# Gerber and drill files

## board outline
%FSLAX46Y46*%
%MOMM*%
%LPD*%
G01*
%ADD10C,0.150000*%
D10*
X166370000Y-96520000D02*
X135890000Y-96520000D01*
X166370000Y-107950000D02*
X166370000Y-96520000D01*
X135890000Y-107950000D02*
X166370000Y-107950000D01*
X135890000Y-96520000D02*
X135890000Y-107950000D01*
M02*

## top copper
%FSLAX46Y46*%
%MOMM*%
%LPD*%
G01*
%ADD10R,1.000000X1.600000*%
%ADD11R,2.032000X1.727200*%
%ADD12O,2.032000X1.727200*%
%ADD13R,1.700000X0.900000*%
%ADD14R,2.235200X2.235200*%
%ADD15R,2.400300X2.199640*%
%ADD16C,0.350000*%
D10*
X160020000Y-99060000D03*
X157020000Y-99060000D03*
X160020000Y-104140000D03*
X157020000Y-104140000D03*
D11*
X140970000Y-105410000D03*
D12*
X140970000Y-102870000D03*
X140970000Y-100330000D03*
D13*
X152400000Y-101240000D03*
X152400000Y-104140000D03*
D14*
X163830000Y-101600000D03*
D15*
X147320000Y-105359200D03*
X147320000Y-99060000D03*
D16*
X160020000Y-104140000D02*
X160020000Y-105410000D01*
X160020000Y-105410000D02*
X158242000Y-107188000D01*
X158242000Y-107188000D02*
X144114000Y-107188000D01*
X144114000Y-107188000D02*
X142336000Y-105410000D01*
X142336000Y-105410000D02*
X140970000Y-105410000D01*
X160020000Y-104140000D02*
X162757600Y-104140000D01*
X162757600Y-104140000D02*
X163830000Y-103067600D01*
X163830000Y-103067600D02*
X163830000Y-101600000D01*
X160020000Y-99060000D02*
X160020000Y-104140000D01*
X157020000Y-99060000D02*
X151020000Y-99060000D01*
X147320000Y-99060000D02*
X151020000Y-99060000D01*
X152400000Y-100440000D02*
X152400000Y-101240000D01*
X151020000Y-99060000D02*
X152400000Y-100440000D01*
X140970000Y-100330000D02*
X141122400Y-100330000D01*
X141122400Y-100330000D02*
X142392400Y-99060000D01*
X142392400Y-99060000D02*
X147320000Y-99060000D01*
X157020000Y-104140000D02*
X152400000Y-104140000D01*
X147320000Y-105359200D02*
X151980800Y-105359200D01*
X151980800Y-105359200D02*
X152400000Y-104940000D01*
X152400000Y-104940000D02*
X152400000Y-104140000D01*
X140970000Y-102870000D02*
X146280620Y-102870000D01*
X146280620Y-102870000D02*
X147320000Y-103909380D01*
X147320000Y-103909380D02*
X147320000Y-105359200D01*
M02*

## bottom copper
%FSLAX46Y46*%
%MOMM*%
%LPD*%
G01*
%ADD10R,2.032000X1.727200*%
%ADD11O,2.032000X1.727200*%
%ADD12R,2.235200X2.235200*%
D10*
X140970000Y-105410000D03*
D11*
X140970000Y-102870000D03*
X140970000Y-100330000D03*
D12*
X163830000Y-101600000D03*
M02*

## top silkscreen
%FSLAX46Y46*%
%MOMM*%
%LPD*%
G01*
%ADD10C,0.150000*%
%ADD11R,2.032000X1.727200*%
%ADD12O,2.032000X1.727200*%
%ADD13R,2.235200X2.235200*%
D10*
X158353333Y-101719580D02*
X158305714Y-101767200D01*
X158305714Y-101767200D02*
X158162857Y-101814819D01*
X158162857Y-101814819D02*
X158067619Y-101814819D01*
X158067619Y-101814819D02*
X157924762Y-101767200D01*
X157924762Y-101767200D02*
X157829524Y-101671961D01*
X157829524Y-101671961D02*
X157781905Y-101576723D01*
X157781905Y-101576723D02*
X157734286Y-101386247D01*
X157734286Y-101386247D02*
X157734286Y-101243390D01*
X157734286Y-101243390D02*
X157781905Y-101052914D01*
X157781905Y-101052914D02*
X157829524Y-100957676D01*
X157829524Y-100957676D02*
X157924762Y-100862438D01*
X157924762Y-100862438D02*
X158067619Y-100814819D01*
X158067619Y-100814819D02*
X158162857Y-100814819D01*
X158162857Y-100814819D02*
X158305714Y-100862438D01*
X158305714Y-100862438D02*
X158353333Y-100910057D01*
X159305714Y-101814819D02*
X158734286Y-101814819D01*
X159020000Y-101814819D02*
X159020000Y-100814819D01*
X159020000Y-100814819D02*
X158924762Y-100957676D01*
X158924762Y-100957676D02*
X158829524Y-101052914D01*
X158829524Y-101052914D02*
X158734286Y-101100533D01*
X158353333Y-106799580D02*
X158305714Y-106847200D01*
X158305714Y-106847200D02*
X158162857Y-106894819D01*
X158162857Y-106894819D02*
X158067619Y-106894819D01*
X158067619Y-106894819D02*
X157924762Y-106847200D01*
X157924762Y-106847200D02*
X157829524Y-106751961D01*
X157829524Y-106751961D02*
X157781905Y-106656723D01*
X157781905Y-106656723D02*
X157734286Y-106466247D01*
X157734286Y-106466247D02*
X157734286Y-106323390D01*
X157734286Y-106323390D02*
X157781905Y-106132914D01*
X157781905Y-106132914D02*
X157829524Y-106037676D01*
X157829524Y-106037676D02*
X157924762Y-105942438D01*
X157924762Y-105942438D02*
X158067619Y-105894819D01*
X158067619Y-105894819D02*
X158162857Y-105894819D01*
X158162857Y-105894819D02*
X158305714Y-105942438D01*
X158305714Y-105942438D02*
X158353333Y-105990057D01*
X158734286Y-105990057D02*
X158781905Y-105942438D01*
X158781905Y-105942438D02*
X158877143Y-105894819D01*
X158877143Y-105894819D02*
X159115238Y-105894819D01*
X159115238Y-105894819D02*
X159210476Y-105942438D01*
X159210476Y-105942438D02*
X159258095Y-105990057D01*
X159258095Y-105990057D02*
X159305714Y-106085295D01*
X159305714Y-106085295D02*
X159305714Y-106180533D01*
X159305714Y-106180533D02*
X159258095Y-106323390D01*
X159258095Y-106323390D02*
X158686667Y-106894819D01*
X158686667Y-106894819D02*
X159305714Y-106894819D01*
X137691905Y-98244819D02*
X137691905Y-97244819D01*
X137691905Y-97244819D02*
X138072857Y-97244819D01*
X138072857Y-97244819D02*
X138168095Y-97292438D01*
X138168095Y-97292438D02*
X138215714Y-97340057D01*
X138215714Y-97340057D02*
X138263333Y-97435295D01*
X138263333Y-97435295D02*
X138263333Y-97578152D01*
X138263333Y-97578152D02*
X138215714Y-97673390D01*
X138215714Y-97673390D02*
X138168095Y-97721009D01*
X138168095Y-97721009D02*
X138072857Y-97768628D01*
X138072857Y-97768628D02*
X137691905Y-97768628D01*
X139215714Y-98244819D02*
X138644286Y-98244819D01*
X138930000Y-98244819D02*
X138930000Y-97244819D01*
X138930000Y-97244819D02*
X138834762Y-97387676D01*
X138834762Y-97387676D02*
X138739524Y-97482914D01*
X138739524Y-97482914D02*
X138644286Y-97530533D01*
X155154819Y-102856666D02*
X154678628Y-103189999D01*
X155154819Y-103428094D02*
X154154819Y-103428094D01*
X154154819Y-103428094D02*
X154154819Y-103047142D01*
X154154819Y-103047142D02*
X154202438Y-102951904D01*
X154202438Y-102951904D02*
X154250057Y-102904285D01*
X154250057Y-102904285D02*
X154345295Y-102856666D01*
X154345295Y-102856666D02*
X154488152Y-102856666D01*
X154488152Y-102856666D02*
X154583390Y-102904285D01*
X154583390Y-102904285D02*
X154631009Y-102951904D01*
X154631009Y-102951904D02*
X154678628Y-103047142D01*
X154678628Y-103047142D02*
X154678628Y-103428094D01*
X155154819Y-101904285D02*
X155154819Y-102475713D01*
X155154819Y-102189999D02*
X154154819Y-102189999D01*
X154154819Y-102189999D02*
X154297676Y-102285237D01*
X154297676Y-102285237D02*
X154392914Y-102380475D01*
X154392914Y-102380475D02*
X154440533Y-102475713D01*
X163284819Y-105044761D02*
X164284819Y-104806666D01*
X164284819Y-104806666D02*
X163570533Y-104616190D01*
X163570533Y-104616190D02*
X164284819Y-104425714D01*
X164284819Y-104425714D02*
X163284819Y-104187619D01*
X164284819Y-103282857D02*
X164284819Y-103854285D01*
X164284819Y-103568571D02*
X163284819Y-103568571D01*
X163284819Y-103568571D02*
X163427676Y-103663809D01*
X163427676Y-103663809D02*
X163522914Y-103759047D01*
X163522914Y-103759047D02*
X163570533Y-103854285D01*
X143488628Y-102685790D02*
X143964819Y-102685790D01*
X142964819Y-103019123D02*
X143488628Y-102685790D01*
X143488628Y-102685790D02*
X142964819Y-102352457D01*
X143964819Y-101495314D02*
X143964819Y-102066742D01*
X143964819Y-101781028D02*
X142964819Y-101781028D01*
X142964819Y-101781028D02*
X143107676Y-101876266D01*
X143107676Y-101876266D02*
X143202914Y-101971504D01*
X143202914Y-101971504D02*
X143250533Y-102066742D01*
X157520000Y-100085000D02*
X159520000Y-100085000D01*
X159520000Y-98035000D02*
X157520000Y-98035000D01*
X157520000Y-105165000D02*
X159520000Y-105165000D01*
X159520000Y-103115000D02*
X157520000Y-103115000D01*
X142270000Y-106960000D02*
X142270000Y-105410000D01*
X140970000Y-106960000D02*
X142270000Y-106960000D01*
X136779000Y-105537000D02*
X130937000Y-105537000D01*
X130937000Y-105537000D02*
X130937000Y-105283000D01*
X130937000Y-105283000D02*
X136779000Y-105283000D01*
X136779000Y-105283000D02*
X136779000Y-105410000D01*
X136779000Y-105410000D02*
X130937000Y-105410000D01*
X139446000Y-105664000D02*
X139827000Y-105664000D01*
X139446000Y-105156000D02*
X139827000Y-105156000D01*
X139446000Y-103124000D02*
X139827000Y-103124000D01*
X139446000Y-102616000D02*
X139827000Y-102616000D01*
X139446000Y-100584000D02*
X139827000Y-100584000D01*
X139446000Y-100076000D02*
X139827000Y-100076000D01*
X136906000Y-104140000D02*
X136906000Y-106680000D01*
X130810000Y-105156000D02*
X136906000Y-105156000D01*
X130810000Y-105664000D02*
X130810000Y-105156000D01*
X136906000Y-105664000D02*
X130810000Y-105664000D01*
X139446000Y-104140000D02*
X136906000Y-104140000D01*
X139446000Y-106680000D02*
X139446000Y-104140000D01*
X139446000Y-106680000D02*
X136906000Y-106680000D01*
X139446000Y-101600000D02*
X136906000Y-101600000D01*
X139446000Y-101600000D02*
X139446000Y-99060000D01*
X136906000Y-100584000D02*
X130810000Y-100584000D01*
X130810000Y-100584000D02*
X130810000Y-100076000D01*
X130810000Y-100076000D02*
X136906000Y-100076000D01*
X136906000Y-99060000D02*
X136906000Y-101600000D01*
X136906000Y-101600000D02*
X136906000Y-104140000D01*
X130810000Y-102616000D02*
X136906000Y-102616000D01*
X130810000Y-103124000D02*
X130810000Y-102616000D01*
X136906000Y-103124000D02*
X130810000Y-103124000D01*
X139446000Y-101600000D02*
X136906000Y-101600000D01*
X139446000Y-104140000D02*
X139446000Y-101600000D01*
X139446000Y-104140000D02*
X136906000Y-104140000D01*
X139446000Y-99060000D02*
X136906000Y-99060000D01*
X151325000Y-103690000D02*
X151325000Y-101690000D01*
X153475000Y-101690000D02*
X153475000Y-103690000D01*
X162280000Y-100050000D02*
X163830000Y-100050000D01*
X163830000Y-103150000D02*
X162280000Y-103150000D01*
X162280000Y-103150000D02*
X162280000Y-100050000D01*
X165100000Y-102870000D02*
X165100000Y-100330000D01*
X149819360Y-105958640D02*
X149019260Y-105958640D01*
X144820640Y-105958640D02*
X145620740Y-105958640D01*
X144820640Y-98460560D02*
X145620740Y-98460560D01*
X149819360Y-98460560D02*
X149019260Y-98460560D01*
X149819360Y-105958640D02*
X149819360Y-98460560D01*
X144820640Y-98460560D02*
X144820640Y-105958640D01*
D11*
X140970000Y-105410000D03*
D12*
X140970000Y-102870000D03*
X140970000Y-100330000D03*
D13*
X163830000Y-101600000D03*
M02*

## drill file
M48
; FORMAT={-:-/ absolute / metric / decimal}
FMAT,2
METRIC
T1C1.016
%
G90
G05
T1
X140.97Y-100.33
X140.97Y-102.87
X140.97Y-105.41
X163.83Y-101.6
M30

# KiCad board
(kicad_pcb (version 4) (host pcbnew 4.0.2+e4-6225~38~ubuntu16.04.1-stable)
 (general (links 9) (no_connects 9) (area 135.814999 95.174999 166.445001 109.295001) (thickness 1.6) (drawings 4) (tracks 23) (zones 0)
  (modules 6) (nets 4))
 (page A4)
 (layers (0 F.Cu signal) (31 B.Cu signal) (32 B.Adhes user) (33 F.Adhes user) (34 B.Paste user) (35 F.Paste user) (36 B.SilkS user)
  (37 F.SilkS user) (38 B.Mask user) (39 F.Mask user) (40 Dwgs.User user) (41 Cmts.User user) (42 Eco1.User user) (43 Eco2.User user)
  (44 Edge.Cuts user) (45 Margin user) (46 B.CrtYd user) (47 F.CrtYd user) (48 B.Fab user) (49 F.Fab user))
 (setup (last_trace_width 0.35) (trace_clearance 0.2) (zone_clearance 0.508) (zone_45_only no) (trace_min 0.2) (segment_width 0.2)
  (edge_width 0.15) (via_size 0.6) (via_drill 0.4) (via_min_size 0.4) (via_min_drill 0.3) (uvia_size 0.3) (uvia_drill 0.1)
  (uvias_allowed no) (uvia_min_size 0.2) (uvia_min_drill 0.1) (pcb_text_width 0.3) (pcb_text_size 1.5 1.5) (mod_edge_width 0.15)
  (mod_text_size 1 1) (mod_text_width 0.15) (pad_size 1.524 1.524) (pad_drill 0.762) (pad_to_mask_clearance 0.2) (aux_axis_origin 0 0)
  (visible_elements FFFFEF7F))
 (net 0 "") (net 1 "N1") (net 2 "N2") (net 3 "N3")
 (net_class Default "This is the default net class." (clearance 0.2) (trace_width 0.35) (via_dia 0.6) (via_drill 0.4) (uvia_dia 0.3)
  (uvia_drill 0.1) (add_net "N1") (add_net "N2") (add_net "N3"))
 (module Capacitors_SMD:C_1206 (layer F.Cu) (at 158.52 99.06 180)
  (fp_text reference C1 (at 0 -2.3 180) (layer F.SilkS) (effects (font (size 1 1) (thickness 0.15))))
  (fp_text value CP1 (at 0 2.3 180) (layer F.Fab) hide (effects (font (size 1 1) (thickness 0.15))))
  (fp_line (start 1 -1.025) (end -1 -1.025) (layer F.SilkS) (width 0.15))
  (fp_line (start -1 1.025) (end 1 1.025) (layer F.SilkS) (width 0.15))
  (pad 1 smd rect (at -1.5 0 180) (size 1 1.6) (layers F.Cu F.Paste F.Mask) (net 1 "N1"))
  (pad 2 smd rect (at 1.5 0 180) (size 1 1.6) (layers F.Cu F.Paste F.Mask) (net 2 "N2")))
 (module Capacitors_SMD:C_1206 (layer F.Cu) (at 158.52 104.14 180)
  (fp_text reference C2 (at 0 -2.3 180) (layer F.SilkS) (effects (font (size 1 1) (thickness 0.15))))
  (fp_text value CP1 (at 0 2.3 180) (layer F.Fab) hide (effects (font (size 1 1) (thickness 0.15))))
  (fp_line (start 1 -1.025) (end -1 -1.025) (layer F.SilkS) (width 0.15))
  (fp_line (start -1 1.025) (end 1 1.025) (layer F.SilkS) (width 0.15))
  (pad 1 smd rect (at -1.5 0 180) (size 1 1.6) (layers F.Cu F.Paste F.Mask) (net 1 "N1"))
  (pad 2 smd rect (at 1.5 0 180) (size 1 1.6) (layers F.Cu F.Paste F.Mask) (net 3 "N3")))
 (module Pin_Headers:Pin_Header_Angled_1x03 (layer F.Cu) (at 140.97 105.41 180)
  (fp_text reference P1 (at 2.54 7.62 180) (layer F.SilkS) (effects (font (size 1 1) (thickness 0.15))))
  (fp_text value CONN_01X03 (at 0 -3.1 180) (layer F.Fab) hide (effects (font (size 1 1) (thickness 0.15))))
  (fp_line (start -1.3 -1.55) (end -1.3 0) (layer F.SilkS) (width 0.15))
  (fp_line (start 0 -1.55) (end -1.3 -1.55) (layer F.SilkS) (width 0.15))
  (fp_line (start 4.191 -0.127) (end 10.033 -0.127) (layer F.SilkS) (width 0.15))
  (fp_line (start 10.033 -0.127) (end 10.033 0.127) (layer F.SilkS) (width 0.15))
  (fp_line (start 10.033 0.127) (end 4.191 0.127) (layer F.SilkS) (width 0.15))
  (fp_line (start 4.191 0.127) (end 4.191 0) (layer F.SilkS) (width 0.15))
  (fp_line (start 4.191 0) (end 10.033 0) (layer F.SilkS) (width 0.15))
  (fp_line (start 1.524 -0.254) (end 1.143 -0.254) (layer F.SilkS) (width 0.15))
  (fp_line (start 1.524 0.254) (end 1.143 0.254) (layer F.SilkS) (width 0.15))
  (fp_line (start 1.524 2.286) (end 1.143 2.286) (layer F.SilkS) (width 0.15))
  (fp_line (start 1.524 2.794) (end 1.143 2.794) (layer F.SilkS) (width 0.15))
  (fp_line (start 1.524 4.826) (end 1.143 4.826) (layer F.SilkS) (width 0.15))
  (fp_line (start 1.524 5.334) (end 1.143 5.334) (layer F.SilkS) (width 0.15))
  (fp_line (start 4.064 1.27) (end 4.064 -1.27) (layer F.SilkS) (width 0.15))
  (fp_line (start 10.16 0.254) (end 4.064 0.254) (layer F.SilkS) (width 0.15))
  (fp_line (start 10.16 -0.254) (end 10.16 0.254) (layer F.SilkS) (width 0.15))
  (fp_line (start 4.064 -0.254) (end 10.16 -0.254) (layer F.SilkS) (width 0.15))
  (fp_line (start 1.524 1.27) (end 4.064 1.27) (layer F.SilkS) (width 0.15))
  (fp_line (start 1.524 -1.27) (end 1.524 1.27) (layer F.SilkS) (width 0.15))
  (fp_line (start 1.524 -1.27) (end 4.064 -1.27) (layer F.SilkS) (width 0.15))
  (fp_line (start 1.524 3.81) (end 4.064 3.81) (layer F.SilkS) (width 0.15))
  (fp_line (start 1.524 3.81) (end 1.524 6.35) (layer F.SilkS) (width 0.15))
  (fp_line (start 4.064 4.826) (end 10.16 4.826) (layer F.SilkS) (width 0.15))
  (fp_line (start 10.16 4.826) (end 10.16 5.334) (layer F.SilkS) (width 0.15))
  (fp_line (start 10.16 5.334) (end 4.064 5.334) (layer F.SilkS) (width 0.15))
  (fp_line (start 4.064 6.35) (end 4.064 3.81) (layer F.SilkS) (width 0.15))
  (fp_line (start 4.064 3.81) (end 4.064 1.27) (layer F.SilkS) (width 0.15))
  (fp_line (start 10.16 2.794) (end 4.064 2.794) (layer F.SilkS) (width 0.15))
  (fp_line (start 10.16 2.286) (end 10.16 2.794) (layer F.SilkS) (width 0.15))
  (fp_line (start 4.064 2.286) (end 10.16 2.286) (layer F.SilkS) (width 0.15))
  (fp_line (start 1.524 3.81) (end 4.064 3.81) (layer F.SilkS) (width 0.15))
  (fp_line (start 1.524 1.27) (end 1.524 3.81) (layer F.SilkS) (width 0.15))
  (fp_line (start 1.524 1.27) (end 4.064 1.27) (layer F.SilkS) (width 0.15))
  (fp_line (start 1.524 6.35) (end 4.064 6.35) (layer F.SilkS) (width 0.15))
  (pad 1 thru_hole rect (at 0 0 180) (size 2.032 1.7272) (drill 1.016) (layers *.Cu *.Mask F.SilkS) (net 1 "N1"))
  (pad 2 thru_hole oval (at 0 2.54 180) (size 2.032 1.7272) (drill 1.016) (layers *.Cu *.Mask F.SilkS) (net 3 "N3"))
  (pad 3 thru_hole oval (at 0 5.08 180) (size 2.032 1.7272) (drill 1.016) (layers *.Cu *.Mask F.SilkS) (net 2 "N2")))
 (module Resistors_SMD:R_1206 (layer F.Cu) (at 152.4 102.69 270)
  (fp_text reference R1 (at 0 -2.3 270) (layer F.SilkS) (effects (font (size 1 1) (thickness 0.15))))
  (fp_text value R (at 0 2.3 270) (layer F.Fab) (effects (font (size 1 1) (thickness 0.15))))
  (fp_line (start 1 1.075) (end -1 1.075) (layer F.SilkS) (width 0.15))
  (fp_line (start -1 -1.075) (end 1 -1.075) (layer F.SilkS) (width 0.15))
  (pad 1 smd rect (at -1.45 0 270) (size 0.9 1.7) (layers F.Cu F.Paste F.Mask) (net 2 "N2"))
  (pad 2 smd rect (at 1.45 0 270) (size 0.9 1.7) (layers F.Cu F.Paste F.Mask) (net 3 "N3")))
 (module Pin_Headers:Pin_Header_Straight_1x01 (layer F.Cu) (at 163.83 101.6 90)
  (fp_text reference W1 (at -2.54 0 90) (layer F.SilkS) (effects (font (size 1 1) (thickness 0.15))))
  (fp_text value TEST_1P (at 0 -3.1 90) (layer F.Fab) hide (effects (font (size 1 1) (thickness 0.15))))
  (fp_line (start 1.55 -1.55) (end 1.55 0) (layer F.SilkS) (width 0.15))
  (fp_line (start -1.55 0) (end -1.55 -1.55) (layer F.SilkS) (width 0.15))
  (fp_line (start -1.55 -1.55) (end 1.55 -1.55) (layer F.SilkS) (width 0.15))
  (fp_line (start -1.27 1.27) (end 1.27 1.27) (layer F.SilkS) (width 0.15))
  (pad 1 thru_hole rect (at 0 0 90) (size 2.2352 2.2352) (drill 1.016) (layers *.Cu *.Mask F.SilkS) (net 1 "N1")))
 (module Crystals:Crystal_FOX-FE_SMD (layer F.Cu) (at 147.32 102.2096 90)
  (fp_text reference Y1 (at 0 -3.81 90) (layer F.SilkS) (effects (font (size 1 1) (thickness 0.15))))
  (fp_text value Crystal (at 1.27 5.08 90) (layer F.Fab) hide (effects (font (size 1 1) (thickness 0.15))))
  (fp_line (start -3.74904 2.49936) (end -3.74904 1.69926) (layer F.SilkS) (width 0.15))
  (fp_line (start -3.74904 -2.49936) (end -3.74904 -1.69926) (layer F.SilkS) (width 0.15))
  (fp_line (start 3.74904 -2.49936) (end 3.74904 -1.69926) (layer F.SilkS) (width 0.15))
  (fp_line (start 3.74904 2.49936) (end 3.74904 1.69926) (layer F.SilkS) (width 0.15))
  (fp_line (start -3.74904 2.49936) (end 3.74904 2.49936) (layer F.SilkS) (width 0.15))
  (fp_line (start 3.74904 -2.49936) (end -3.74904 -2.49936) (layer F.SilkS) (width 0.15))
  (pad 1 smd rect (at -3.1496 0 90) (size 2.19964 2.4003) (layers F.Cu F.Paste F.Mask) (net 3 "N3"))
  (pad 2 smd rect (at 3.1496 0 90) (size 2.19964 2.4003) (layers F.Cu F.Paste F.Mask) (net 2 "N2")))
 (gr_line (start 166.37 96.52) (end 135.89 96.52) (layer Edge.Cuts) (width 0.15))
 (gr_line (start 166.37 107.95) (end 166.37 96.52) (layer Edge.Cuts) (width 0.15))
 (gr_line (start 135.89 107.95) (end 166.37 107.95) (layer Edge.Cuts) (width 0.15))
 (gr_line (start 135.89 96.52) (end 135.89 107.95) (layer Edge.Cuts) (width 0.15))
 (segment (start 160.02 104.14) (end 160.02 105.41) (width 0.35) (layer F.Cu) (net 1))
 (segment (start 160.02 105.41) (end 158.242 107.188) (width 0.35) (layer F.Cu) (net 1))
 (segment (start 158.242 107.188) (end 144.114 107.188) (width 0.35) (layer F.Cu) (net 1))
 (segment (start 144.114 107.188) (end 142.336 105.41) (width 0.35) (layer F.Cu) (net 1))
 (segment (start 142.336 105.41) (end 140.97 105.41) (width 0.35) (layer F.Cu) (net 1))
 (segment (start 160.02 104.14) (end 162.7576 104.14) (width 0.35) (layer F.Cu) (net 1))
 (segment (start 162.7576 104.14) (end 163.83 103.0676) (width 0.35) (layer F.Cu) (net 1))
 (segment (start 163.83 103.0676) (end 163.83 101.6) (width 0.35) (layer F.Cu) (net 1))
 (segment (start 160.02 99.06) (end 160.02 104.14) (width 0.35) (layer F.Cu) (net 1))
 (segment (start 157.02 99.06) (end 151.02 99.06) (width 0.35) (layer F.Cu) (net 2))
 (segment (start 147.32 99.06) (end 151.02 99.06) (width 0.35) (layer F.Cu) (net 2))
 (segment (start 152.4 100.44) (end 152.4 101.24) (width 0.35) (layer F.Cu) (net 2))
 (segment (start 151.02 99.06) (end 152.4 100.44) (width 0.35) (layer F.Cu) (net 2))
 (segment (start 140.97 100.33) (end 141.1224 100.33) (width 0.35) (layer F.Cu) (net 2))
 (segment (start 141.1224 100.33) (end 142.3924 99.06) (width 0.35) (layer F.Cu) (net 2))
 (segment (start 142.3924 99.06) (end 147.32 99.06) (width 0.35) (layer F.Cu) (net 2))
 (segment (start 157.02 104.14) (end 152.4 104.14) (width 0.35) (layer F.Cu) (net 3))
 (segment (start 147.32 105.3592) (end 151.9808 105.3592) (width 0.35) (layer F.Cu) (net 3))
 (segment (start 151.9808 105.3592) (end 152.4 104.94) (width 0.35) (layer F.Cu) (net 3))
 (segment (start 152.4 104.94) (end 152.4 104.14) (width 0.35) (layer F.Cu) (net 3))
 (segment (start 140.97 102.87) (end 146.28062 102.87) (width 0.35) (layer F.Cu) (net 3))
 (segment (start 146.28062 102.87) (end 147.32 103.90938) (width 0.35) (layer F.Cu) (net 3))
 (segment (start 147.32 103.90938) (end 147.32 105.3592) (width 0.35) (layer F.Cu) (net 3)))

